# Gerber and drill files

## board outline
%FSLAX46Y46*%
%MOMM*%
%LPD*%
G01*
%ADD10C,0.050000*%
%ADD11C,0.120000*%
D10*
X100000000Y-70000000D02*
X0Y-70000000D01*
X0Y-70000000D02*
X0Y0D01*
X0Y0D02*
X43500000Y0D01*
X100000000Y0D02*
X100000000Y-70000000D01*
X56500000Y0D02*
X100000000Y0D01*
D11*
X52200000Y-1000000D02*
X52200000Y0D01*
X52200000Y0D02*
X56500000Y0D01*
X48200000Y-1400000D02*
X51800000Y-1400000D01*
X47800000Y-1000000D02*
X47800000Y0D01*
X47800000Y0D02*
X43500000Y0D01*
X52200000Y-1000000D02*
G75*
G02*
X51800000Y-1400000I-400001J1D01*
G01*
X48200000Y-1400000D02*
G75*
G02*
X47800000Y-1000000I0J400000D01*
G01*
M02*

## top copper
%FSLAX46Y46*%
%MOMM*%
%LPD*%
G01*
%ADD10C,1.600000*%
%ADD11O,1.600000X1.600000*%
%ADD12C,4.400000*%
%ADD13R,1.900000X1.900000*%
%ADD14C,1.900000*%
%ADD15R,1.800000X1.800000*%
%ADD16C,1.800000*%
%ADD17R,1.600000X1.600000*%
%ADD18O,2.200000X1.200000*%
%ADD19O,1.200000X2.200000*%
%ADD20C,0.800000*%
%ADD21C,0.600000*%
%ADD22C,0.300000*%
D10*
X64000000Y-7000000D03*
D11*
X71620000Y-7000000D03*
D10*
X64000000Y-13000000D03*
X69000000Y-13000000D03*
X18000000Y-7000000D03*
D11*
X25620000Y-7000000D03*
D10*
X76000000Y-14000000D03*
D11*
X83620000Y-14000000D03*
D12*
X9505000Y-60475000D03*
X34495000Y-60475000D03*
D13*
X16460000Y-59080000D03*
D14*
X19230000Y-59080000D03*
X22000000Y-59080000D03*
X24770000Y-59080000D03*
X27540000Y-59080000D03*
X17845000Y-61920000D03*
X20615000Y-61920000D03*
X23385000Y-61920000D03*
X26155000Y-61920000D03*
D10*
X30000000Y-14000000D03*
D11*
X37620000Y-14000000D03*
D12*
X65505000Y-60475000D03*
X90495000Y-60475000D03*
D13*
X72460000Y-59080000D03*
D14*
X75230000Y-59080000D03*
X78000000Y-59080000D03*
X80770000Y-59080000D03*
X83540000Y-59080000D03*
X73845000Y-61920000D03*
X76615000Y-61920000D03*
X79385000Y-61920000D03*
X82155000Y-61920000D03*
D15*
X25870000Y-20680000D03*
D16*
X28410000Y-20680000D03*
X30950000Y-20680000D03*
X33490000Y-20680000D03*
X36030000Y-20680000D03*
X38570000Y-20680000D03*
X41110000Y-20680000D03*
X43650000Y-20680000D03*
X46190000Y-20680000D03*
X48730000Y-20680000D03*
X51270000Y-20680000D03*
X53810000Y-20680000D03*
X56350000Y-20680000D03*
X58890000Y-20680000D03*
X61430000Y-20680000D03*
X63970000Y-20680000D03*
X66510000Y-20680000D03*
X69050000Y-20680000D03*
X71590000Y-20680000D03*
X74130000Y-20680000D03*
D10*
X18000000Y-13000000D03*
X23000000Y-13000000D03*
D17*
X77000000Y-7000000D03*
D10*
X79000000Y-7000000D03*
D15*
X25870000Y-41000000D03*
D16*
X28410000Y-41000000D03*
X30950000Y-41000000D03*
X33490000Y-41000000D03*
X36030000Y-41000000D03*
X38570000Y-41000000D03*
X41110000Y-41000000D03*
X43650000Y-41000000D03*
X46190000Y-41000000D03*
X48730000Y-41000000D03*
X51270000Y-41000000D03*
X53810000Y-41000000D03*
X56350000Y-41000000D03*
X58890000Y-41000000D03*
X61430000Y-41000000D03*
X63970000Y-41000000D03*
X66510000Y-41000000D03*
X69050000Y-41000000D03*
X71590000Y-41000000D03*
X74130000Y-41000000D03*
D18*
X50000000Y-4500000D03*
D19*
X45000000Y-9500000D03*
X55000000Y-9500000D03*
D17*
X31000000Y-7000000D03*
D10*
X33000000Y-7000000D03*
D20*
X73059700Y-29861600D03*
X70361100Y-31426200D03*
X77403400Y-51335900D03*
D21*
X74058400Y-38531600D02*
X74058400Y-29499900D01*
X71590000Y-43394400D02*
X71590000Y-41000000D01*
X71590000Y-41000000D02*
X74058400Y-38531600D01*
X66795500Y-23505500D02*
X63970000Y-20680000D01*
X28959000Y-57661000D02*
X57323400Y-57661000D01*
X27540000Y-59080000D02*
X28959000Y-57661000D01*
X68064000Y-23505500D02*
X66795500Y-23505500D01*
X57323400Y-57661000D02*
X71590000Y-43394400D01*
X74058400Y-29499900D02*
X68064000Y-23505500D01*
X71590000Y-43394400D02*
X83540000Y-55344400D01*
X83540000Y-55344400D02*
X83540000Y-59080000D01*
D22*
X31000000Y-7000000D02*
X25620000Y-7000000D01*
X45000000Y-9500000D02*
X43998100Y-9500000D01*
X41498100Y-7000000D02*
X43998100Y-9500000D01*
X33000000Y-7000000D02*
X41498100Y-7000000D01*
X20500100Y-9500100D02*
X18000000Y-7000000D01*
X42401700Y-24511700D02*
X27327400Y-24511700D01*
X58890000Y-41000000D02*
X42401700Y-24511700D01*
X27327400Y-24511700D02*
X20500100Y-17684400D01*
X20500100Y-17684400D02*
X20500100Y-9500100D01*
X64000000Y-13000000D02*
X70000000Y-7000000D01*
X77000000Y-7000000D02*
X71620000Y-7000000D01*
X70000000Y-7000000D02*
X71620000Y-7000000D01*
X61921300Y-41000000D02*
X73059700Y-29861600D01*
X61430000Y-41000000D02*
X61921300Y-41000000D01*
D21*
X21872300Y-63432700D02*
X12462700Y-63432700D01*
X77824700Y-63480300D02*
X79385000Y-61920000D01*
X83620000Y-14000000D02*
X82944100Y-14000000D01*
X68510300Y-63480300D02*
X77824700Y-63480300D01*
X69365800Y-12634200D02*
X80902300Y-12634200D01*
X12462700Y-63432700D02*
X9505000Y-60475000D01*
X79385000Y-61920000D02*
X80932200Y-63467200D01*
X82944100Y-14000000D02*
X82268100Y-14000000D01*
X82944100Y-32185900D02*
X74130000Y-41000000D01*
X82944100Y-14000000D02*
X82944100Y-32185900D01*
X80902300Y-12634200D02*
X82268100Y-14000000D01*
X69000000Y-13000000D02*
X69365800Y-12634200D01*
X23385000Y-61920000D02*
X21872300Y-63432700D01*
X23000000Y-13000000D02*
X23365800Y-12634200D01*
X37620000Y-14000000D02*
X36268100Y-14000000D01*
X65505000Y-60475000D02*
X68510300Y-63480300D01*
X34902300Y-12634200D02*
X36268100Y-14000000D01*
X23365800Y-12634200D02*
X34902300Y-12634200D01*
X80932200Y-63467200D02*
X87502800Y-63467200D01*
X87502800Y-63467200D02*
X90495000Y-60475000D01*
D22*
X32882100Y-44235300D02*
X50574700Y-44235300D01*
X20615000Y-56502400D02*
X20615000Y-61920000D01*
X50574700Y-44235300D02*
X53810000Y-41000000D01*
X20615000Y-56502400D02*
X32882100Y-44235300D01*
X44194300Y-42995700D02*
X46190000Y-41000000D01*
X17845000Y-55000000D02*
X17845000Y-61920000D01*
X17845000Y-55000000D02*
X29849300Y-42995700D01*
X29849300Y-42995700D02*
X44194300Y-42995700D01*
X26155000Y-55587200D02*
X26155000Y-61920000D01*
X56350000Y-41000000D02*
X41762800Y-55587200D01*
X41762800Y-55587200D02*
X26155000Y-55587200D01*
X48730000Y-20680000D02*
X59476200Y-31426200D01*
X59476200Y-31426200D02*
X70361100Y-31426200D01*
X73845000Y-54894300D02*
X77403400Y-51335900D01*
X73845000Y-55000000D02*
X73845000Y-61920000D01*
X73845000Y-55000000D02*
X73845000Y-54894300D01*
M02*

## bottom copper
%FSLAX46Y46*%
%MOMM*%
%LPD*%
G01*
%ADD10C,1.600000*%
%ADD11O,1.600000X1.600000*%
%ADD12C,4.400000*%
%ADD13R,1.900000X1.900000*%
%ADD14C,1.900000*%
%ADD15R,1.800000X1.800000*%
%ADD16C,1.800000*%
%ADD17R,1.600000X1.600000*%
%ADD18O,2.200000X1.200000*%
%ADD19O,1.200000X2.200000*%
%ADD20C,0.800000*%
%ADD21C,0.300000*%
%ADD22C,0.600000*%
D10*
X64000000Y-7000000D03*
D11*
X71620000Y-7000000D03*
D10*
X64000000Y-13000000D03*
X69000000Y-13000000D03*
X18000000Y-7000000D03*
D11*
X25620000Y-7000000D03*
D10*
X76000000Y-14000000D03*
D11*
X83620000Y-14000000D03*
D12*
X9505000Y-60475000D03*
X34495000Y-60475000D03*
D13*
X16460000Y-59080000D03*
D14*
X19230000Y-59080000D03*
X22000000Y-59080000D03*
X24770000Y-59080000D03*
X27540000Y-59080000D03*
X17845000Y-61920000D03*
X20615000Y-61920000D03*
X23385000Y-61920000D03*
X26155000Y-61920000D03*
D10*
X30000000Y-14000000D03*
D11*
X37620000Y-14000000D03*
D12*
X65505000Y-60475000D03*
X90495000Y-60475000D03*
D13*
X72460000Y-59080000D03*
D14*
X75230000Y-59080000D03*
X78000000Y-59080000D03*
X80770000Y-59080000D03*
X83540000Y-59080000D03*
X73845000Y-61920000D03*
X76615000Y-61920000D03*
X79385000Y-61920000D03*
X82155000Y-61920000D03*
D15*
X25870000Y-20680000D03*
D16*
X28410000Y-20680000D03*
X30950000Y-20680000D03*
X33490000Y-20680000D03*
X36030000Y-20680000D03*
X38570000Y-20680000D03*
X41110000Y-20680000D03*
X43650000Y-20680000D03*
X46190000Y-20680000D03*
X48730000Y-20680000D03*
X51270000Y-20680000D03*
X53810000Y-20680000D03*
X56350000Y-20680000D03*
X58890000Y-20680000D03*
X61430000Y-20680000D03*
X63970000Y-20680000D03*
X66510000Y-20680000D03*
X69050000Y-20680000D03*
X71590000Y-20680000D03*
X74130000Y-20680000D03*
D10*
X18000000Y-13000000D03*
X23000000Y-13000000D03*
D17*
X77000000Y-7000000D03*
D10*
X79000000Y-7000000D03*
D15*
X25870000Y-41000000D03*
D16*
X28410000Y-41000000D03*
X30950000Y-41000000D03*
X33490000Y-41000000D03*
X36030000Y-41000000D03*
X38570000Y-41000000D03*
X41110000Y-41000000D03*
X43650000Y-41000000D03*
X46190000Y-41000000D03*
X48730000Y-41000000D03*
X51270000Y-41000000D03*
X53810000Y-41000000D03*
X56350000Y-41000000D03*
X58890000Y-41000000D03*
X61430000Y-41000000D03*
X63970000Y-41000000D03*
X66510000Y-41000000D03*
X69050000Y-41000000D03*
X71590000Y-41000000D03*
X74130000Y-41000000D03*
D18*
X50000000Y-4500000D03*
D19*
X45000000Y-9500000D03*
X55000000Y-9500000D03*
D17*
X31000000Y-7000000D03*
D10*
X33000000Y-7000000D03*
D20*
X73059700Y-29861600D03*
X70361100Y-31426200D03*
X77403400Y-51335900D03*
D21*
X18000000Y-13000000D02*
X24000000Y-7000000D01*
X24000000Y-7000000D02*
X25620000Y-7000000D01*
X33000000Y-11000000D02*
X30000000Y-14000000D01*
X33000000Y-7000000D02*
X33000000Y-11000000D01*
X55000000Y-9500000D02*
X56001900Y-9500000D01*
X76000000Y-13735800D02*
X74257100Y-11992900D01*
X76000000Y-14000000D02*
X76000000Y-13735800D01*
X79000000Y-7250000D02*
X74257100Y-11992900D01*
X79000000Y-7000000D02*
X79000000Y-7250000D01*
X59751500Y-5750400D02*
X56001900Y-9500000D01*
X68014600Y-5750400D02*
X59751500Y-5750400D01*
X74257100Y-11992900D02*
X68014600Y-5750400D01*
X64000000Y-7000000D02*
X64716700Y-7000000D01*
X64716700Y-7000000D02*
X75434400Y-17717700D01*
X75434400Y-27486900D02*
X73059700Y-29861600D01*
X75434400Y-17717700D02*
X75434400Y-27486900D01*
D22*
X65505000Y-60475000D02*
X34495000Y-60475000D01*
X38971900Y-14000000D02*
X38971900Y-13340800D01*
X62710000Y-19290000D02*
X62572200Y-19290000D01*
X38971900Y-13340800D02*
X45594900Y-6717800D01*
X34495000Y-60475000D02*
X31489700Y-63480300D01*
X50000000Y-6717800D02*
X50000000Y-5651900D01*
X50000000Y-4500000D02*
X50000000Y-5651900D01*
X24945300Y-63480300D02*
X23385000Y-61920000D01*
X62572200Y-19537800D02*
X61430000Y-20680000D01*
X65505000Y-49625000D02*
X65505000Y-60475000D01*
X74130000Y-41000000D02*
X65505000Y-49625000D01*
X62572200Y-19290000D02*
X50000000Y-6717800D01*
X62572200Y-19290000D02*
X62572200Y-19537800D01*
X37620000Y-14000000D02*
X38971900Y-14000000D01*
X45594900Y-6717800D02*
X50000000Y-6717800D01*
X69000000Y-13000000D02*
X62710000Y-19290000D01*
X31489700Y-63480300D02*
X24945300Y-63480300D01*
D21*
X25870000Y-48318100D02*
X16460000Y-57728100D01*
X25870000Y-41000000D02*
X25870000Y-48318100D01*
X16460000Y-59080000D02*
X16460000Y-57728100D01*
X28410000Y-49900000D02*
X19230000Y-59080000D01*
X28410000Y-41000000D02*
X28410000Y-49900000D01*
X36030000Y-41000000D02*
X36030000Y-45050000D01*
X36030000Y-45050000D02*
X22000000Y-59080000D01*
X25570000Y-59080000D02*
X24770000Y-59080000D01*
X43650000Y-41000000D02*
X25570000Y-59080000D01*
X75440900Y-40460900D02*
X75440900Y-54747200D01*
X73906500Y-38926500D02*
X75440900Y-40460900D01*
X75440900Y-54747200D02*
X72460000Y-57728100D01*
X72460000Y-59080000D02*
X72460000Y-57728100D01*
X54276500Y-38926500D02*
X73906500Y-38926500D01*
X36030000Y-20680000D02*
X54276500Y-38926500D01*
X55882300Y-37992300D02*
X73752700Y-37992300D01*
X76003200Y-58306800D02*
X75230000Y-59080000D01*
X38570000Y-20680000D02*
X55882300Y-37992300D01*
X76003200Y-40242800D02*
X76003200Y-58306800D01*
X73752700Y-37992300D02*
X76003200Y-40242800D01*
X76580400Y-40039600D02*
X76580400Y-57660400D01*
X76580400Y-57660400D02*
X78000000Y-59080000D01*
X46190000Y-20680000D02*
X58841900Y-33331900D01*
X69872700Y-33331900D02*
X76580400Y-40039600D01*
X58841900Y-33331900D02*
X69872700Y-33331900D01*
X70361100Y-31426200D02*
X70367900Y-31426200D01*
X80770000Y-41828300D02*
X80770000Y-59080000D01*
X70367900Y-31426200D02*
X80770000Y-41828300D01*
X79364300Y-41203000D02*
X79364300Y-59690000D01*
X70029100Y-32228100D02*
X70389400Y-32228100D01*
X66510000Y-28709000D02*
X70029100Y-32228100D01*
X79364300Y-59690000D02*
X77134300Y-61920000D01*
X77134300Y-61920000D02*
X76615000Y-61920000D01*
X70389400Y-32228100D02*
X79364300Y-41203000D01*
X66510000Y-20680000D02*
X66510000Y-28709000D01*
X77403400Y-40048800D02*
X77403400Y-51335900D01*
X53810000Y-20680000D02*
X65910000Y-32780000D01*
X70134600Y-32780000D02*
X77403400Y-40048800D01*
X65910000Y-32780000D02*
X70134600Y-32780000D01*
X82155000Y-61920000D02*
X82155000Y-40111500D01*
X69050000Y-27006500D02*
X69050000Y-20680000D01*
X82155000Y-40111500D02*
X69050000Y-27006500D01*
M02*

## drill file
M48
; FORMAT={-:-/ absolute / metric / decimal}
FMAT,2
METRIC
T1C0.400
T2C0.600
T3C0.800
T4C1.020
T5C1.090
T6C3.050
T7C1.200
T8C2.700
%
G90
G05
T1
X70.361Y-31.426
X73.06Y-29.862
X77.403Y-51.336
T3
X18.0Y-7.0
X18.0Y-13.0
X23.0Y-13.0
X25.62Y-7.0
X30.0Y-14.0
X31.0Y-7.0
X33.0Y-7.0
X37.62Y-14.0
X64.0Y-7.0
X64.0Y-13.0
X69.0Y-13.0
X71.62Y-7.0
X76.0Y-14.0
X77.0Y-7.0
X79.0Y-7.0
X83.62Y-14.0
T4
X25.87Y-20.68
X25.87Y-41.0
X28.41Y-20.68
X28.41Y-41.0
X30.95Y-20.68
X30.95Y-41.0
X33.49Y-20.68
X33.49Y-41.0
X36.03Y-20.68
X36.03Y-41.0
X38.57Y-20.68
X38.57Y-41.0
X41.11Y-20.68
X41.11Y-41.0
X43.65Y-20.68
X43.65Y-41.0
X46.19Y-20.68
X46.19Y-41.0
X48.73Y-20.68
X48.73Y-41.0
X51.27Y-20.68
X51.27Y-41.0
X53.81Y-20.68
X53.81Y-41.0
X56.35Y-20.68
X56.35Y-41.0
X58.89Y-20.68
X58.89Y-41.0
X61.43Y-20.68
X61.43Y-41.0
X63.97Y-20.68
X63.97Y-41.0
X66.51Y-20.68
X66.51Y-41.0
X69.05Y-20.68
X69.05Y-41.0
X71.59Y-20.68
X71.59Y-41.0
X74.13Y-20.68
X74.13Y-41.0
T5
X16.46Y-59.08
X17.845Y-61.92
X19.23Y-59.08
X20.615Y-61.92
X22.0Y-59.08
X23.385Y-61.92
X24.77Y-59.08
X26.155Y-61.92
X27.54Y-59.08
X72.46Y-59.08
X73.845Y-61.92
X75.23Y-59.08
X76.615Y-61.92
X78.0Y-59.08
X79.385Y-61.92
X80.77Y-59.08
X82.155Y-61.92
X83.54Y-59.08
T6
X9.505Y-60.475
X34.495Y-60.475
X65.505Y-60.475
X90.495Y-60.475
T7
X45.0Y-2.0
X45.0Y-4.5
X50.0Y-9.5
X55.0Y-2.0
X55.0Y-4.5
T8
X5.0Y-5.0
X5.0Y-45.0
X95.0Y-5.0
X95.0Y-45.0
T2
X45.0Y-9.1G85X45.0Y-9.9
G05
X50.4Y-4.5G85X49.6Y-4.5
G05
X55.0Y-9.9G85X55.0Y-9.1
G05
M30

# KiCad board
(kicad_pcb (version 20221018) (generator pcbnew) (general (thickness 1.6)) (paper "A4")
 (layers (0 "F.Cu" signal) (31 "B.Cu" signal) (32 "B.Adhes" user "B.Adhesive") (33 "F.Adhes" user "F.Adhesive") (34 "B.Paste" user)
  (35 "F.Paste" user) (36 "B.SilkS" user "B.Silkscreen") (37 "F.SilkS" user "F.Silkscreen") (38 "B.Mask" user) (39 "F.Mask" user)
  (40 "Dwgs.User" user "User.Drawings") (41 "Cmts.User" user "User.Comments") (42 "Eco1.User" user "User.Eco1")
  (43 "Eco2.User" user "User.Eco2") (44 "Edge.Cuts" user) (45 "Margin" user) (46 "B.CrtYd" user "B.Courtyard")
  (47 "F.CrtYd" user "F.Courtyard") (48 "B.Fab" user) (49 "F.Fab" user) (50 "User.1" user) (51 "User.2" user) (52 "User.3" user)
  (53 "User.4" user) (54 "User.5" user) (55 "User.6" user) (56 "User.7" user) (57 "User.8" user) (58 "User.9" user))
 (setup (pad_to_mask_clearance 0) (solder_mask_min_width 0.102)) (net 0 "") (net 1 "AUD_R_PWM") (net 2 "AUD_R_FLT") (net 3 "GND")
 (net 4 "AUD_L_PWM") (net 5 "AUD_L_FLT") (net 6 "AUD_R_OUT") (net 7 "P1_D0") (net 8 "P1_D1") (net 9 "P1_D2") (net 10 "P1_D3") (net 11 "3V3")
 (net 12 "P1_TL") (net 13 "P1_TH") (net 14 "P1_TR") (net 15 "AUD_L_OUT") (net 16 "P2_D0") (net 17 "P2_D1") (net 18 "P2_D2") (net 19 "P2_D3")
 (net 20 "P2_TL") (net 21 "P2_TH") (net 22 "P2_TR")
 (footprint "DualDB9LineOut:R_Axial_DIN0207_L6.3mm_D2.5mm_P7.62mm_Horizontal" (layer "F.Cu") (at 64 7)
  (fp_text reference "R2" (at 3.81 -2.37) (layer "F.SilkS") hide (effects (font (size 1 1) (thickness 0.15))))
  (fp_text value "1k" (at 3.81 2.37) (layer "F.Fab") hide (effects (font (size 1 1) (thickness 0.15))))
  (pad "1" thru_hole circle (at 0 0) (size 1.6 1.6) (drill 0.8) (layers "*.Cu" "*.Mask") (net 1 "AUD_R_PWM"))
  (pad "2" thru_hole oval (at 7.62 0) (size 1.6 1.6) (drill 0.8) (layers "*.Cu" "*.Mask") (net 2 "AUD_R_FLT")))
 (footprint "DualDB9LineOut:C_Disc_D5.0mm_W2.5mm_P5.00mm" (layer "F.Cu") (at 64 13)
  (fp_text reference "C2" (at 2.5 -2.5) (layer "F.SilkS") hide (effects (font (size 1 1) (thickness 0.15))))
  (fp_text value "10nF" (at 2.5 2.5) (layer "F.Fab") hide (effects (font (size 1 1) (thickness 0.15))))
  (pad "1" thru_hole circle (at 0 0) (size 1.6 1.6) (drill 0.8) (layers "*.Cu" "*.Mask") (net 2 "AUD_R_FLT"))
  (pad "2" thru_hole circle (at 5 0) (size 1.6 1.6) (drill 0.8) (layers "*.Cu" "*.Mask") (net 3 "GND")))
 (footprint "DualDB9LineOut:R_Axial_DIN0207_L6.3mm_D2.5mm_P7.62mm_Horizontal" (layer "F.Cu") (at 18 7)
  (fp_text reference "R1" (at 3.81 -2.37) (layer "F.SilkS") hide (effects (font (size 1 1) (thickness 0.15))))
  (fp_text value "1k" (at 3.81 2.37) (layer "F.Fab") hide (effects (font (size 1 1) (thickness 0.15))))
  (pad "1" thru_hole circle (at 0 0) (size 1.6 1.6) (drill 0.8) (layers "*.Cu" "*.Mask") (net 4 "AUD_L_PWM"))
  (pad "2" thru_hole oval (at 7.62 0) (size 1.6 1.6) (drill 0.8) (layers "*.Cu" "*.Mask") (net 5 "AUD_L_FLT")))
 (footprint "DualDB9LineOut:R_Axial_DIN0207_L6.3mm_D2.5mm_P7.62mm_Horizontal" (layer "F.Cu") (at 76 14)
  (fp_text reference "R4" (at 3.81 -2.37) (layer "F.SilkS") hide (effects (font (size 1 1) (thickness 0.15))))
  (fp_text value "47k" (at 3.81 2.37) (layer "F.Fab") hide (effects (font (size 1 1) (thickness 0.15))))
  (pad "1" thru_hole circle (at 0 0) (size 1.6 1.6) (drill 0.8) (layers "*.Cu" "*.Mask") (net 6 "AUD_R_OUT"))
  (pad "2" thru_hole oval (at 7.62 0) (size 1.6 1.6) (drill 0.8) (layers "*.Cu" "*.Mask") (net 3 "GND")))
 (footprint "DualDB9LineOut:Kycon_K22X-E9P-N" (layer "F.Cu") (at 16.46 59.08)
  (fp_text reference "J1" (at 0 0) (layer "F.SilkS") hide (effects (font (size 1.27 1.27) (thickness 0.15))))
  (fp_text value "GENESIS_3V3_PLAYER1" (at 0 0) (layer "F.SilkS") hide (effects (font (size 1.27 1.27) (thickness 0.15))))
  (pad "0" thru_hole circle (at -6.955 1.395) (size 4.4 4.4) (drill 3.05) (layers "F&B.Cu" "*.Mask") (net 3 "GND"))
  (pad "0" thru_hole circle (at 18.035 1.395) (size 4.4 4.4) (drill 3.05) (layers "F&B.Cu" "*.Mask") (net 3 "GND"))
  (pad "1" thru_hole rect (at 0 0) (size 1.9 1.9) (drill 1.09) (layers "F&B.Cu" "*.Mask") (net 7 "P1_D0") (thermal_bridge_angle 45))
  (pad "2" thru_hole circle (at 2.77 0) (size 1.9 1.9) (drill 1.09) (layers "F&B.Cu" "*.Mask") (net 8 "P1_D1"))
  (pad "3" thru_hole circle (at 5.54 0) (size 1.9 1.9) (drill 1.09) (layers "F&B.Cu" "*.Mask") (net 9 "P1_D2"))
  (pad "4" thru_hole circle (at 8.31 0) (size 1.9 1.9) (drill 1.09) (layers "F&B.Cu" "*.Mask") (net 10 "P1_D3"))
  (pad "5" thru_hole circle (at 11.08 0) (size 1.9 1.9) (drill 1.09) (layers "F&B.Cu" "*.Mask") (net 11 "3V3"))
  (pad "6" thru_hole circle (at 1.385 2.84) (size 1.9 1.9) (drill 1.09) (layers "F&B.Cu" "*.Mask") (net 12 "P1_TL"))
  (pad "7" thru_hole circle (at 4.155 2.84) (size 1.9 1.9) (drill 1.09) (layers "F&B.Cu" "*.Mask") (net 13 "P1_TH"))
  (pad "8" thru_hole circle (at 6.925 2.84) (size 1.9 1.9) (drill 1.09) (layers "F&B.Cu" "*.Mask") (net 3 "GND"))
  (pad "9" thru_hole circle (at 9.695 2.84) (size 1.9 1.9) (drill 1.09) (layers "F&B.Cu" "*.Mask") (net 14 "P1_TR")))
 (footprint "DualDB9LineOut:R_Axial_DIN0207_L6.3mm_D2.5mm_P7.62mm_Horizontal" (layer "F.Cu") (at 30 14)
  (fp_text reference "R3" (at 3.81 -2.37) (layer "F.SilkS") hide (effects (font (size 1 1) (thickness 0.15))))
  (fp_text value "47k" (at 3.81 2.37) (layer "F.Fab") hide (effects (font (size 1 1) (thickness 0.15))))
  (pad "1" thru_hole circle (at 0 0) (size 1.6 1.6) (drill 0.8) (layers "*.Cu" "*.Mask") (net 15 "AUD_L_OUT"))
  (pad "2" thru_hole oval (at 7.62 0) (size 1.6 1.6) (drill 0.8) (layers "*.Cu" "*.Mask") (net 3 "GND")))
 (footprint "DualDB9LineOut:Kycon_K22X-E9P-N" (layer "F.Cu") (at 72.46 59.08)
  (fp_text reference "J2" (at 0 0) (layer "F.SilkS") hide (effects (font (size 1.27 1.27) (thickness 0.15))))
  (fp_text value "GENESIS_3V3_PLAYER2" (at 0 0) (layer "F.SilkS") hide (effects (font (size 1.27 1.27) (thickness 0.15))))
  (pad "0" thru_hole circle (at -6.955 1.395) (size 4.4 4.4) (drill 3.05) (layers "F&B.Cu" "*.Mask") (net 3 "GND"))
  (pad "0" thru_hole circle (at 18.035 1.395) (size 4.4 4.4) (drill 3.05) (layers "F&B.Cu" "*.Mask") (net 3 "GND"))
  (pad "1" thru_hole rect (at 0 0) (size 1.9 1.9) (drill 1.09) (layers "F&B.Cu" "*.Mask") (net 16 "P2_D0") (thermal_bridge_angle 45))
  (pad "2" thru_hole circle (at 2.77 0) (size 1.9 1.9) (drill 1.09) (layers "F&B.Cu" "*.Mask") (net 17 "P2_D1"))
  (pad "3" thru_hole circle (at 5.54 0) (size 1.9 1.9) (drill 1.09) (layers "F&B.Cu" "*.Mask") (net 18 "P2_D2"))
  (pad "4" thru_hole circle (at 8.31 0) (size 1.9 1.9) (drill 1.09) (layers "F&B.Cu" "*.Mask") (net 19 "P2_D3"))
  (pad "5" thru_hole circle (at 11.08 0) (size 1.9 1.9) (drill 1.09) (layers "F&B.Cu" "*.Mask") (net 11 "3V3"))
  (pad "6" thru_hole circle (at 1.385 2.84) (size 1.9 1.9) (drill 1.09) (layers "F&B.Cu" "*.Mask") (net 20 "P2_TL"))
  (pad "7" thru_hole circle (at 4.155 2.84) (size 1.9 1.9) (drill 1.09) (layers "F&B.Cu" "*.Mask") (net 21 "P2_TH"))
  (pad "8" thru_hole circle (at 6.925 2.84) (size 1.9 1.9) (drill 1.09) (layers "F&B.Cu" "*.Mask") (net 3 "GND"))
  (pad "9" thru_hole circle (at 9.695 2.84) (size 1.9 1.9) (drill 1.09) (layers "F&B.Cu" "*.Mask") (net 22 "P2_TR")))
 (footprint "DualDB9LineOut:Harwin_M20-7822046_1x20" (layer "F.Cu") (at 25.87 20.68 90)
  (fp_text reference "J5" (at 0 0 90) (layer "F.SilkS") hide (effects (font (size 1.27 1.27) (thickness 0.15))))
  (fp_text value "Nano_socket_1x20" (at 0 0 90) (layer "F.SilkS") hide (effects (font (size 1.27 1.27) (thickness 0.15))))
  (pad "1" thru_hole rect (at 0 0 90) (size 1.8 1.8) (drill 1.02) (layers "F&B.Cu" "*.Mask") (thermal_bridge_angle 45))
  (pad "2" thru_hole circle (at 0 2.54 90) (size 1.8 1.8) (drill 1.02) (layers "F&B.Cu" "*.Mask"))
  (pad "3" thru_hole circle (at 0 5.08 90) (size 1.8 1.8) (drill 1.02) (layers "F&B.Cu" "*.Mask"))
  (pad "4" thru_hole circle (at 0 7.62 90) (size 1.8 1.8) (drill 1.02) (layers "F&B.Cu" "*.Mask"))
  (pad "5" thru_hole circle (at 0 10.16 90) (size 1.8 1.8) (drill 1.02) (layers "F&B.Cu" "*.Mask") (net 16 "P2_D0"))
  (pad "6" thru_hole circle (at 0 12.7 90) (size 1.8 1.8) (drill 1.02) (layers "F&B.Cu" "*.Mask") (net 17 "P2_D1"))
  (pad "7" thru_hole circle (at 0 15.24 90) (size 1.8 1.8) (drill 1.02) (layers "F&B.Cu" "*.Mask"))
  (pad "8" thru_hole circle (at 0 17.78 90) (size 1.8 1.8) (drill 1.02) (layers "F&B.Cu" "*.Mask"))
  (pad "9" thru_hole circle (at 0 20.32 90) (size 1.8 1.8) (drill 1.02) (layers "F&B.Cu" "*.Mask") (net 18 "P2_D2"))
  (pad "10" thru_hole circle (at 0 22.86 90) (size 1.8 1.8) (drill 1.02) (layers "F&B.Cu" "*.Mask") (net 19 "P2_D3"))
  (pad "11" thru_hole circle (at 0 25.4 90) (size 1.8 1.8) (drill 1.02) (layers "F&B.Cu" "*.Mask"))
  (pad "12" thru_hole circle (at 0 27.94 90) (size 1.8 1.8) (drill 1.02) (layers "F&B.Cu" "*.Mask") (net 20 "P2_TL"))
  (pad "13" thru_hole circle (at 0 30.48 90) (size 1.8 1.8) (drill 1.02) (layers "F&B.Cu" "*.Mask"))
  (pad "14" thru_hole circle (at 0 33.02 90) (size 1.8 1.8) (drill 1.02) (layers "F&B.Cu" "*.Mask"))
  (pad "15" thru_hole circle (at 0 35.56 90) (size 1.8 1.8) (drill 1.02) (layers "F&B.Cu" "*.Mask") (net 3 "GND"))
  (pad "16" thru_hole circle (at 0 38.1 90) (size 1.8 1.8) (drill 1.02) (layers "F&B.Cu" "*.Mask") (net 11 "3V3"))
  (pad "17" thru_hole circle (at 0 40.64 90) (size 1.8 1.8) (drill 1.02) (layers "F&B.Cu" "*.Mask") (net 21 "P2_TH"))
  (pad "18" thru_hole circle (at 0 43.18 90) (size 1.8 1.8) (drill 1.02) (layers "F&B.Cu" "*.Mask") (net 22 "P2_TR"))
  (pad "19" thru_hole circle (at 0 45.72 90) (size 1.8 1.8) (drill 1.02) (layers "F&B.Cu" "*.Mask"))
  (pad "20" thru_hole circle (at 0 48.26 90) (size 1.8 1.8) (drill 1.02) (layers "F&B.Cu" "*.Mask")))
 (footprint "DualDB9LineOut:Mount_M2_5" (layer "F.Cu") (at 5 5)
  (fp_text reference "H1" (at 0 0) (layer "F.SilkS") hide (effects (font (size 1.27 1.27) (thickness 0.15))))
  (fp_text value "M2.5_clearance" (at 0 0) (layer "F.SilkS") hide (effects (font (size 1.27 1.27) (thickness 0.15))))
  (pad "" np_thru_hole circle (at 0 0) (size 2.7 2.7) (drill 2.7) (layers "F&B.Cu" "*.Mask")))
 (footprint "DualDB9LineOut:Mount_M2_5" (layer "F.Cu") (at 5 45)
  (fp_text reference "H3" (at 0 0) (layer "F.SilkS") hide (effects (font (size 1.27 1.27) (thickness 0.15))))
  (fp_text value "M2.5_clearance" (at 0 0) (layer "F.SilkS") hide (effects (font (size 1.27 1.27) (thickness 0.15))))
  (pad "" np_thru_hole circle (at 0 0) (size 2.7 2.7) (drill 2.7) (layers "F&B.Cu" "*.Mask")))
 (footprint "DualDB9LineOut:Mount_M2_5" (layer "F.Cu") (at 95 5)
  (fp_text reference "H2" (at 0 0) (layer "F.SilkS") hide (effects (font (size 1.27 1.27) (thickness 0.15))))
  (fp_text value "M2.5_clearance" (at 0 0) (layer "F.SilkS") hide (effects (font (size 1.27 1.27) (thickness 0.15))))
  (pad "" np_thru_hole circle (at 0 0) (size 2.7 2.7) (drill 2.7) (layers "F&B.Cu" "*.Mask")))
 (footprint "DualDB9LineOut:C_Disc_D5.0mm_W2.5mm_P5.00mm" (layer "F.Cu") (at 18 13)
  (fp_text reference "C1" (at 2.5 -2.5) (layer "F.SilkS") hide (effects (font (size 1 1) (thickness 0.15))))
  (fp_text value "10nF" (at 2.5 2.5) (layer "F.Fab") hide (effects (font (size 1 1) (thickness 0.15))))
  (pad "1" thru_hole circle (at 0 0) (size 1.6 1.6) (drill 0.8) (layers "*.Cu" "*.Mask") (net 5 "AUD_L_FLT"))
  (pad "2" thru_hole circle (at 5 0) (size 1.6 1.6) (drill 0.8) (layers "*.Cu" "*.Mask") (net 3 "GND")))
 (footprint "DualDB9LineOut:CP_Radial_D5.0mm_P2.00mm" (layer "F.Cu") (at 77 7)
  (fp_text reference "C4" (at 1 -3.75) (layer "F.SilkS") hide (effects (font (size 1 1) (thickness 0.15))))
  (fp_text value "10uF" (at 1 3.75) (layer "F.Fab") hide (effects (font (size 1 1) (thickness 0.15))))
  (pad "1" thru_hole rect (at 0 0) (size 1.6 1.6) (drill 0.8) (layers "*.Cu" "*.Mask") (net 2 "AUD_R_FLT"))
  (pad "2" thru_hole circle (at 2 0) (size 1.6 1.6) (drill 0.8) (layers "*.Cu" "*.Mask") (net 6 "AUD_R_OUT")))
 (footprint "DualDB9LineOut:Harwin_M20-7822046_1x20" (layer "F.Cu") (at 25.87 41 90)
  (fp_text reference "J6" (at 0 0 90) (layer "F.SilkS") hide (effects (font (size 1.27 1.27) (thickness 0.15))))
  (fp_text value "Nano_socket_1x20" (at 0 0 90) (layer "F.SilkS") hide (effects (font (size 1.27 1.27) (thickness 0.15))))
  (pad "1" thru_hole rect (at 0 0 90) (size 1.8 1.8) (drill 1.02) (layers "F&B.Cu" "*.Mask") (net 7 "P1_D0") (thermal_bridge_angle 45))
  (pad "2" thru_hole circle (at 0 2.54 90) (size 1.8 1.8) (drill 1.02) (layers "F&B.Cu" "*.Mask") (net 8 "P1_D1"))
  (pad "3" thru_hole circle (at 0 5.08 90) (size 1.8 1.8) (drill 1.02) (layers "F&B.Cu" "*.Mask"))
  (pad "4" thru_hole circle (at 0 7.62 90) (size 1.8 1.8) (drill 1.02) (layers "F&B.Cu" "*.Mask"))
  (pad "5" thru_hole circle (at 0 10.16 90) (size 1.8 1.8) (drill 1.02) (layers "F&B.Cu" "*.Mask") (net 9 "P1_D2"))
  (pad "6" thru_hole circle (at 0 12.7 90) (size 1.8 1.8) (drill 1.02) (layers "F&B.Cu" "*.Mask"))
  (pad "7" thru_hole circle (at 0 15.24 90) (size 1.8 1.8) (drill 1.02) (layers "F&B.Cu" "*.Mask"))
  (pad "8" thru_hole circle (at 0 17.78 90) (size 1.8 1.8) (drill 1.02) (layers "F&B.Cu" "*.Mask") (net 10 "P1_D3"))
  (pad "9" thru_hole circle (at 0 20.32 90) (size 1.8 1.8) (drill 1.02) (layers "F&B.Cu" "*.Mask") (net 12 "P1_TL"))
  (pad "10" thru_hole circle (at 0 22.86 90) (size 1.8 1.8) (drill 1.02) (layers "F&B.Cu" "*.Mask"))
  (pad "11" thru_hole circle (at 0 25.4 90) (size 1.8 1.8) (drill 1.02) (layers "F&B.Cu" "*.Mask"))
  (pad "12" thru_hole circle (at 0 27.94 90) (size 1.8 1.8) (drill 1.02) (layers "F&B.Cu" "*.Mask") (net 13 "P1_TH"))
  (pad "13" thru_hole circle (at 0 30.48 90) (size 1.8 1.8) (drill 1.02) (layers "F&B.Cu" "*.Mask") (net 14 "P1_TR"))
  (pad "14" thru_hole circle (at 0 33.02 90) (size 1.8 1.8) (drill 1.02) (layers "F&B.Cu" "*.Mask") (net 4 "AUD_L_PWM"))
  (pad "15" thru_hole circle (at 0 35.56 90) (size 1.8 1.8) (drill 1.02) (layers "F&B.Cu" "*.Mask") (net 1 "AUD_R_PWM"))
  (pad "16" thru_hole circle (at 0 38.1 90) (size 1.8 1.8) (drill 1.02) (layers "F&B.Cu" "*.Mask"))
  (pad "17" thru_hole circle (at 0 40.64 90) (size 1.8 1.8) (drill 1.02) (layers "F&B.Cu" "*.Mask"))
  (pad "18" thru_hole circle (at 0 43.18 90) (size 1.8 1.8) (drill 1.02) (layers "F&B.Cu" "*.Mask"))
  (pad "19" thru_hole circle (at 0 45.72 90) (size 1.8 1.8) (drill 1.02) (layers "F&B.Cu" "*.Mask") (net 11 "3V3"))
  (pad "20" thru_hole circle (at 0 48.26 90) (size 1.8 1.8) (drill 1.02) (layers "F&B.Cu" "*.Mask") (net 3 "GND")))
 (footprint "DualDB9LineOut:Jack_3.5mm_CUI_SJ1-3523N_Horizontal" (layer "F.Cu") (at 50 4.5 180)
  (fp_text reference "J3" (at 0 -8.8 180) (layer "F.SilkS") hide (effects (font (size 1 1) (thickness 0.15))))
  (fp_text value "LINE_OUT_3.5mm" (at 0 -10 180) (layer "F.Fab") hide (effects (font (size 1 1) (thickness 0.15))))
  (fp_line (start -2.2 3.5) (end -2.2 4.5) (stroke (width 0.12) (type solid)) (layer "Edge.Cuts"))
  (fp_line (start -2.2 4.5) (end -6.5 4.5) (stroke (width 0.12) (type solid)) (layer "Edge.Cuts"))
  (fp_line (start 1.8 3.1) (end -1.8 3.1) (stroke (width 0.12) (type solid)) (layer "Edge.Cuts"))
  (fp_line (start 2.2 3.5) (end 2.2 4.5) (stroke (width 0.12) (type solid)) (layer "Edge.Cuts"))
  (fp_line (start 2.2 4.5) (end 6.5 4.5) (stroke (width 0.12) (type solid)) (layer "Edge.Cuts"))
  (fp_arc (start -2.2 3.5) (mid -2.082843 3.217158) (end -1.8 3.1) (stroke (width 0.12) (type solid)) (layer "Edge.Cuts"))
  (fp_arc (start 1.8 3.1) (mid 2.082843 3.217157) (end 2.2 3.5) (stroke (width 0.12) (type solid)) (layer "Edge.Cuts"))
  (pad "" np_thru_hole circle (at -5 0 180) (size 1.2 1.2) (drill 1.2) (layers "F&B.Cu" "*.Mask"))
  (pad "" np_thru_hole circle (at -5 2.5 180) (size 1.2 1.2) (drill 1.2) (layers "F&B.Cu" "*.Mask"))
  (pad "" np_thru_hole circle (at 0 -5 180) (size 1.2 1.2) (drill 1.2) (layers "F&B.Cu" "*.Mask"))
  (pad "" np_thru_hole circle (at 5 0 180) (size 1.2 1.2) (drill 1.2) (layers "F&B.Cu" "*.Mask"))
  (pad "" np_thru_hole circle (at 5 2.5 180) (size 1.2 1.2) (drill 1.2) (layers "F&B.Cu" "*.Mask"))
  (pad "1" thru_hole oval (at 0 0 180) (size 2.2 1.2) (drill oval 1.4 0.6) (layers "*.Cu" "*.Mask") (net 3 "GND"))
  (pad "2" thru_hole oval (at 5 -5) (size 1.2 2.2) (drill oval 0.6 1.4) (layers "*.Cu" "*.Mask") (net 15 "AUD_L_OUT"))
  (pad "3" thru_hole oval (at -5 -5 180) (size 1.2 2.2) (drill oval 0.6 1.4) (layers "*.Cu" "*.Mask") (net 6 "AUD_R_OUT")))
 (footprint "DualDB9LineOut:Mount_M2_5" (layer "F.Cu") (at 95 45)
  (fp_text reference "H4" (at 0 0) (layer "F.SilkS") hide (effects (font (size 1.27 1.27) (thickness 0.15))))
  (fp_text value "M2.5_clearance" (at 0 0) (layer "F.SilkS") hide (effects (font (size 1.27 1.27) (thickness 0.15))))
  (pad "" np_thru_hole circle (at 0 0) (size 2.7 2.7) (drill 2.7) (layers "F&B.Cu" "*.Mask")))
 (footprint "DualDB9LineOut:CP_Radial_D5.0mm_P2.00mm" (layer "F.Cu") (at 31 7)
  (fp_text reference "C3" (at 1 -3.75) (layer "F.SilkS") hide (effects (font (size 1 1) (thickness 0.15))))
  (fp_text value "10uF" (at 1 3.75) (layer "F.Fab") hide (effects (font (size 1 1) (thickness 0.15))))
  (pad "1" thru_hole rect (at 0 0) (size 1.6 1.6) (drill 0.8) (layers "*.Cu" "*.Mask") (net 5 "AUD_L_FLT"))
  (pad "2" thru_hole circle (at 2 0) (size 1.6 1.6) (drill 0.8) (layers "*.Cu" "*.Mask") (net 15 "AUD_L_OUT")))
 (gr_line (start 100 70) (end 0 70) (stroke (width 0.05) (type default)) (layer "Edge.Cuts"))
 (gr_line (start 0 70) (end 0 0) (stroke (width 0.05) (type default)) (layer "Edge.Cuts"))
 (gr_line (start 0 0) (end 43.5 0) (stroke (width 0.05) (type default)) (layer "Edge.Cuts"))
 (gr_line (start 100 0) (end 100 70) (stroke (width 0.05) (type default)) (layer "Edge.Cuts"))
 (gr_line (start 56.5 0) (end 100 0) (stroke (width 0.05) (type default)) (layer "Edge.Cuts"))
 (segment (start 74.0584 38.5316) (end 74.0584 29.4999) (width 0.6) (layer "F.Cu") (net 11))
 (segment (start 71.59 43.3944) (end 71.59 41) (width 0.6) (layer "F.Cu") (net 11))
 (segment (start 71.59 41) (end 74.0584 38.5316) (width 0.6) (layer "F.Cu") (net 11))
 (segment (start 66.7955 23.5055) (end 63.97 20.68) (width 0.6) (layer "F.Cu") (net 11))
 (segment (start 28.959 57.661) (end 57.3234 57.661) (width 0.6) (layer "F.Cu") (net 11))
 (segment (start 27.54 59.08) (end 28.959 57.661) (width 0.6) (layer "F.Cu") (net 11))
 (segment (start 68.064 23.5055) (end 66.7955 23.5055) (width 0.6) (layer "F.Cu") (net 11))
 (segment (start 57.3234 57.661) (end 71.59 43.3944) (width 0.6) (layer "F.Cu") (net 11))
 (segment (start 74.0584 29.4999) (end 68.064 23.5055) (width 0.6) (layer "F.Cu") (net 11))
 (segment (start 71.59 43.3944) (end 83.54 55.3444) (width 0.6) (layer "F.Cu") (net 11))
 (segment (start 83.54 55.3444) (end 83.54 59.08) (width 0.6) (layer "F.Cu") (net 11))
 (segment (start 31 7) (end 25.62 7) (width 0.3) (layer "F.Cu") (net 5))
 (segment (start 18 13) (end 24 7) (width 0.3) (layer "B.Cu") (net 5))
 (segment (start 24 7) (end 25.62 7) (width 0.3) (layer "B.Cu") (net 5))
 (segment (start 45 9.5) (end 43.9981 9.5) (width 0.3) (layer "F.Cu") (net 15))
 (segment (start 41.4981 7) (end 43.9981 9.5) (width 0.3) (layer "F.Cu") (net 15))
 (segment (start 33 7) (end 41.4981 7) (width 0.3) (layer "F.Cu") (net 15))
 (segment (start 33 11) (end 30 14) (width 0.3) (layer "B.Cu") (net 15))
 (segment (start 33 7) (end 33 11) (width 0.3) (layer "B.Cu") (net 15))
 (segment (start 20.5001 9.5001) (end 18 7) (width 0.3) (layer "F.Cu") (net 4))
 (segment (start 42.4017 24.5117) (end 27.3274 24.5117) (width 0.3) (layer "F.Cu") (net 4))
 (segment (start 58.89 41) (end 42.4017 24.5117) (width 0.3) (layer "F.Cu") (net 4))
 (segment (start 27.3274 24.5117) (end 20.5001 17.6844) (width 0.3) (layer "F.Cu") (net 4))
 (segment (start 20.5001 17.6844) (end 20.5001 9.5001) (width 0.3) (layer "F.Cu") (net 4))
 (segment (start 64 13) (end 70 7) (width 0.3) (layer "F.Cu") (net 2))
 (segment (start 77 7) (end 71.62 7) (width 0.3) (layer "F.Cu") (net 2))
 (segment (start 70 7) (end 71.62 7) (width 0.3) (layer "F.Cu") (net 2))
 (segment (start 55 9.5) (end 56.0019 9.5) (width 0.3) (layer "B.Cu") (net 6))
 (segment (start 76 13.7358) (end 74.2571 11.9929) (width 0.3) (layer "B.Cu") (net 6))
 (segment (start 76 14) (end 76 13.7358) (width 0.3) (layer "B.Cu") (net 6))
 (segment (start 79 7.25) (end 74.2571 11.9929) (width 0.3) (layer "B.Cu") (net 6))
 (segment (start 79 7) (end 79 7.25) (width 0.3) (layer "B.Cu") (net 6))
 (segment (start 59.7515 5.7504) (end 56.0019 9.5) (width 0.3) (layer "B.Cu") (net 6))
 (segment (start 68.0146 5.7504) (end 59.7515 5.7504) (width 0.3) (layer "B.Cu") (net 6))
 (segment (start 74.2571 11.9929) (end 68.0146 5.7504) (width 0.3) (layer "B.Cu") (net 6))
 (segment (start 61.9213 41) (end 73.0597 29.8616) (width 0.3) (layer "F.Cu") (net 1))
 (segment (start 61.43 41) (end 61.9213 41) (width 0.3) (layer "F.Cu") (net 1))
 (via (at 73.0597 29.8616) (size 0.8) (drill 0.4) (layers "F.Cu" "B.Cu") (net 1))
 (segment (start 64 7) (end 64.7167 7) (width 0.3) (layer "B.Cu") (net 1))
 (segment (start 64.7167 7) (end 75.4344 17.7177) (width 0.3) (layer "B.Cu") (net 1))
 (segment (start 75.4344 27.4869) (end 73.0597 29.8616) (width 0.3) (layer "B.Cu") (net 1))
 (segment (start 75.4344 17.7177) (end 75.4344 27.4869) (width 0.3) (layer "B.Cu") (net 1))
 (segment (start 21.8723 63.4327) (end 12.4627 63.4327) (width 0.6) (layer "F.Cu") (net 3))
 (segment (start 77.8247 63.4803) (end 79.385 61.92) (width 0.6) (layer "F.Cu") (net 3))
 (segment (start 83.62 14) (end 82.9441 14) (width 0.6) (layer "F.Cu") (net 3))
 (segment (start 68.5103 63.4803) (end 77.8247 63.4803) (width 0.6) (layer "F.Cu") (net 3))
 (segment (start 69.3658 12.6342) (end 80.9023 12.6342) (width 0.6) (layer "F.Cu") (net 3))
 (segment (start 12.4627 63.4327) (end 9.505 60.475) (width 0.6) (layer "F.Cu") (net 3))
 (segment (start 79.385 61.92) (end 80.9322 63.4672) (width 0.6) (layer "F.Cu") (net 3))
 (segment (start 82.9441 14) (end 82.2681 14) (width 0.6) (layer "F.Cu") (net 3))
 (segment (start 82.9441 32.1859) (end 74.13 41) (width 0.6) (layer "F.Cu") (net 3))
 (segment (start 82.9441 14) (end 82.9441 32.1859) (width 0.6) (layer "F.Cu") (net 3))
 (segment (start 80.9023 12.6342) (end 82.2681 14) (width 0.6) (layer "F.Cu") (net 3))
 (segment (start 69 13) (end 69.3658 12.6342) (width 0.6) (layer "F.Cu") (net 3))
 (segment (start 23.385 61.92) (end 21.8723 63.4327) (width 0.6) (layer "F.Cu") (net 3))
 (segment (start 23 13) (end 23.3658 12.6342) (width 0.6) (layer "F.Cu") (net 3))
 (segment (start 37.62 14) (end 36.2681 14) (width 0.6) (layer "F.Cu") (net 3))
 (segment (start 65.505 60.475) (end 68.5103 63.4803) (width 0.6) (layer "F.Cu") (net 3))
 (segment (start 34.9023 12.6342) (end 36.2681 14) (width 0.6) (layer "F.Cu") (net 3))
 (segment (start 23.3658 12.6342) (end 34.9023 12.6342) (width 0.6) (layer "F.Cu") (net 3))
 (segment (start 80.9322 63.4672) (end 87.5028 63.4672) (width 0.6) (layer "F.Cu") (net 3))
 (segment (start 87.5028 63.4672) (end 90.495 60.475) (width 0.6) (layer "F.Cu") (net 3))
 (segment (start 65.505 60.475) (end 34.495 60.475) (width 0.6) (layer "B.Cu") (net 3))
 (segment (start 38.9719 14) (end 38.9719 13.3408) (width 0.6) (layer "B.Cu") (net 3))
 (segment (start 62.71 19.29) (end 62.5722 19.29) (width 0.6) (layer "B.Cu") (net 3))
 (segment (start 38.9719 13.3408) (end 45.5949 6.7178) (width 0.6) (layer "B.Cu") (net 3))
 (segment (start 34.495 60.475) (end 31.4897 63.4803) (width 0.6) (layer "B.Cu") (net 3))
 (segment (start 50 6.7178) (end 50 5.6519) (width 0.6) (layer "B.Cu") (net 3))
 (segment (start 50 4.5) (end 50 5.6519) (width 0.6) (layer "B.Cu") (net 3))
 (segment (start 24.9453 63.4803) (end 23.385 61.92) (width 0.6) (layer "B.Cu") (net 3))
 (segment (start 62.5722 19.5378) (end 61.43 20.68) (width 0.6) (layer "B.Cu") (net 3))
 (segment (start 65.505 49.625) (end 65.505 60.475) (width 0.6) (layer "B.Cu") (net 3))
 (segment (start 74.13 41) (end 65.505 49.625) (width 0.6) (layer "B.Cu") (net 3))
 (segment (start 62.5722 19.29) (end 50 6.7178) (width 0.6) (layer "B.Cu") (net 3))
 (segment (start 62.5722 19.29) (end 62.5722 19.5378) (width 0.6) (layer "B.Cu") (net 3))
 (segment (start 37.62 14) (end 38.9719 14) (width 0.6) (layer "B.Cu") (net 3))
 (segment (start 45.5949 6.7178) (end 50 6.7178) (width 0.6) (layer "B.Cu") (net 3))
 (segment (start 69 13) (end 62.71 19.29) (width 0.6) (layer "B.Cu") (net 3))
 (segment (start 31.4897 63.4803) (end 24.9453 63.4803) (width 0.6) (layer "B.Cu") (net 3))
 (segment (start 25.87 48.3181) (end 16.46 57.7281) (width 0.3) (layer "B.Cu") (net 7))
 (segment (start 25.87 41) (end 25.87 48.3181) (width 0.3) (layer "B.Cu") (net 7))
 (segment (start 16.46 59.08) (end 16.46 57.7281) (width 0.3) (layer "B.Cu") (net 7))
 (segment (start 28.41 49.9) (end 19.23 59.08) (width 0.3) (layer "B.Cu") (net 8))
 (segment (start 28.41 41) (end 28.41 49.9) (width 0.3) (layer "B.Cu") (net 8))
 (segment (start 36.03 41) (end 36.03 45.05) (width 0.3) (layer "B.Cu") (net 9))
 (segment (start 36.03 45.05) (end 22 59.08) (width 0.3) (layer "B.Cu") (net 9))
 (segment (start 25.57 59.08) (end 24.77 59.08) (width 0.3) (layer "B.Cu") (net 10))
 (segment (start 43.65 41) (end 25.57 59.08) (width 0.3) (layer "B.Cu") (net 10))
 (segment (start 32.8821 44.2353) (end 50.5747 44.2353) (width 0.3) (layer "F.Cu") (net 13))
 (segment (start 20.615 56.5024) (end 20.615 61.92) (width 0.3) (layer "F.Cu") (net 13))
 (segment (start 50.5747 44.2353) (end 53.81 41) (width 0.3) (layer "F.Cu") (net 13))
 (segment (start 20.615 56.5024) (end 32.8821 44.2353) (width 0.3) (layer "F.Cu") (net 13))
 (segment (start 44.1943 42.9957) (end 46.19 41) (width 0.3) (layer "F.Cu") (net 12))
 (segment (start 17.845 55) (end 17.845 61.92) (width 0.3) (layer "F.Cu") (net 12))
 (segment (start 17.845 55) (end 29.8493 42.9957) (width 0.3) (layer "F.Cu") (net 12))
 (segment (start 29.8493 42.9957) (end 44.1943 42.9957) (width 0.3) (layer "F.Cu") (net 12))
 (segment (start 26.155 55.5872) (end 26.155 61.92) (width 0.3) (layer "F.Cu") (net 14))
 (segment (start 56.35 41) (end 41.7628 55.5872) (width 0.3) (layer "F.Cu") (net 14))
 (segment (start 41.7628 55.5872) (end 26.155 55.5872) (width 0.3) (layer "F.Cu") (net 14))
 (segment (start 75.4409 40.4609) (end 75.4409 54.7472) (width 0.3) (layer "B.Cu") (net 16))
 (segment (start 73.9065 38.9265) (end 75.4409 40.4609) (width 0.3) (layer "B.Cu") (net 16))
 (segment (start 75.4409 54.7472) (end 72.46 57.7281) (width 0.3) (layer "B.Cu") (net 16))
 (segment (start 72.46 59.08) (end 72.46 57.7281) (width 0.3) (layer "B.Cu") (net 16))
 (segment (start 54.2765 38.9265) (end 73.9065 38.9265) (width 0.3) (layer "B.Cu") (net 16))
 (segment (start 36.03 20.68) (end 54.2765 38.9265) (width 0.3) (layer "B.Cu") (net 16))
 (segment (start 55.8823 37.9923) (end 73.7527 37.9923) (width 0.3) (layer "B.Cu") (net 17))
 (segment (start 76.0032 58.3068) (end 75.23 59.08) (width 0.3) (layer "B.Cu") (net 17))
 (segment (start 38.57 20.68) (end 55.8823 37.9923) (width 0.3) (layer "B.Cu") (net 17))
 (segment (start 76.0032 40.2428) (end 76.0032 58.3068) (width 0.3) (layer "B.Cu") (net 17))
 (segment (start 73.7527 37.9923) (end 76.0032 40.2428) (width 0.3) (layer "B.Cu") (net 17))
 (segment (start 76.5804 40.0396) (end 76.5804 57.6604) (width 0.3) (layer "B.Cu") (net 18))
 (segment (start 76.5804 57.6604) (end 78 59.08) (width 0.3) (layer "B.Cu") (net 18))
 (segment (start 46.19 20.68) (end 58.8419 33.3319) (width 0.3) (layer "B.Cu") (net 18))
 (segment (start 69.8727 33.3319) (end 76.5804 40.0396) (width 0.3) (layer "B.Cu") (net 18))
 (segment (start 58.8419 33.3319) (end 69.8727 33.3319) (width 0.3) (layer "B.Cu") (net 18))
 (segment (start 48.73 20.68) (end 59.4762 31.4262) (width 0.3) (layer "F.Cu") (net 19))
 (segment (start 59.4762 31.4262) (end 70.3611 31.4262) (width 0.3) (layer "F.Cu") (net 19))
 (via (at 70.3611 31.4262) (size 0.8) (drill 0.4) (layers "F.Cu" "B.Cu") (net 19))
 (segment (start 70.3611 31.4262) (end 70.3679 31.4262) (width 0.3) (layer "B.Cu") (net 19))
 (segment (start 80.77 41.8283) (end 80.77 59.08) (width 0.3) (layer "B.Cu") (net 19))
 (segment (start 70.3679 31.4262) (end 80.77 41.8283) (width 0.3) (layer "B.Cu") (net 19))
 (segment (start 79.3643 41.203) (end 79.3643 59.69) (width 0.3) (layer "B.Cu") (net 21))
 (segment (start 70.0291 32.2281) (end 70.3894 32.2281) (width 0.3) (layer "B.Cu") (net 21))
 (segment (start 66.51 28.709) (end 70.0291 32.2281) (width 0.3) (layer "B.Cu") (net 21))
 (segment (start 79.3643 59.69) (end 77.1343 61.92) (width 0.3) (layer "B.Cu") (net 21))
 (segment (start 77.1343 61.92) (end 76.615 61.92) (width 0.3) (layer "B.Cu") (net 21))
 (segment (start 70.3894 32.2281) (end 79.3643 41.203) (width 0.3) (layer "B.Cu") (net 21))
 (segment (start 66.51 20.68) (end 66.51 28.709) (width 0.3) (layer "B.Cu") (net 21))
 (segment (start 73.845 54.8943) (end 77.4034 51.3359) (width 0.3) (layer "F.Cu") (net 20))
 (segment (start 73.845 55) (end 73.845 61.92) (width 0.3) (layer "F.Cu") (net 20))
 (segment (start 73.845 55) (end 73.845 54.8943) (width 0.3) (layer "F.Cu") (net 20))
 (via (at 77.4034 51.3359) (size 0.8) (drill 0.4) (layers "F.Cu" "B.Cu") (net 20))
 (segment (start 77.4034 40.0488) (end 77.4034 51.3359) (width 0.3) (layer "B.Cu") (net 20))
 (segment (start 53.81 20.68) (end 65.91 32.78) (width 0.3) (layer "B.Cu") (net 20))
 (segment (start 70.1346 32.78) (end 77.4034 40.0488) (width 0.3) (layer "B.Cu") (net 20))
 (segment (start 65.91 32.78) (end 70.1346 32.78) (width 0.3) (layer "B.Cu") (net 20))
 (segment (start 82.155 61.92) (end 82.155 40.1115) (width 0.3) (layer "B.Cu") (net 22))
 (segment (start 69.05 27.0065) (end 69.05 20.68) (width 0.3) (layer "B.Cu") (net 22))
 (segment (start 82.155 40.1115) (end 69.05 27.0065) (width 0.3) (layer "B.Cu") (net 22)))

